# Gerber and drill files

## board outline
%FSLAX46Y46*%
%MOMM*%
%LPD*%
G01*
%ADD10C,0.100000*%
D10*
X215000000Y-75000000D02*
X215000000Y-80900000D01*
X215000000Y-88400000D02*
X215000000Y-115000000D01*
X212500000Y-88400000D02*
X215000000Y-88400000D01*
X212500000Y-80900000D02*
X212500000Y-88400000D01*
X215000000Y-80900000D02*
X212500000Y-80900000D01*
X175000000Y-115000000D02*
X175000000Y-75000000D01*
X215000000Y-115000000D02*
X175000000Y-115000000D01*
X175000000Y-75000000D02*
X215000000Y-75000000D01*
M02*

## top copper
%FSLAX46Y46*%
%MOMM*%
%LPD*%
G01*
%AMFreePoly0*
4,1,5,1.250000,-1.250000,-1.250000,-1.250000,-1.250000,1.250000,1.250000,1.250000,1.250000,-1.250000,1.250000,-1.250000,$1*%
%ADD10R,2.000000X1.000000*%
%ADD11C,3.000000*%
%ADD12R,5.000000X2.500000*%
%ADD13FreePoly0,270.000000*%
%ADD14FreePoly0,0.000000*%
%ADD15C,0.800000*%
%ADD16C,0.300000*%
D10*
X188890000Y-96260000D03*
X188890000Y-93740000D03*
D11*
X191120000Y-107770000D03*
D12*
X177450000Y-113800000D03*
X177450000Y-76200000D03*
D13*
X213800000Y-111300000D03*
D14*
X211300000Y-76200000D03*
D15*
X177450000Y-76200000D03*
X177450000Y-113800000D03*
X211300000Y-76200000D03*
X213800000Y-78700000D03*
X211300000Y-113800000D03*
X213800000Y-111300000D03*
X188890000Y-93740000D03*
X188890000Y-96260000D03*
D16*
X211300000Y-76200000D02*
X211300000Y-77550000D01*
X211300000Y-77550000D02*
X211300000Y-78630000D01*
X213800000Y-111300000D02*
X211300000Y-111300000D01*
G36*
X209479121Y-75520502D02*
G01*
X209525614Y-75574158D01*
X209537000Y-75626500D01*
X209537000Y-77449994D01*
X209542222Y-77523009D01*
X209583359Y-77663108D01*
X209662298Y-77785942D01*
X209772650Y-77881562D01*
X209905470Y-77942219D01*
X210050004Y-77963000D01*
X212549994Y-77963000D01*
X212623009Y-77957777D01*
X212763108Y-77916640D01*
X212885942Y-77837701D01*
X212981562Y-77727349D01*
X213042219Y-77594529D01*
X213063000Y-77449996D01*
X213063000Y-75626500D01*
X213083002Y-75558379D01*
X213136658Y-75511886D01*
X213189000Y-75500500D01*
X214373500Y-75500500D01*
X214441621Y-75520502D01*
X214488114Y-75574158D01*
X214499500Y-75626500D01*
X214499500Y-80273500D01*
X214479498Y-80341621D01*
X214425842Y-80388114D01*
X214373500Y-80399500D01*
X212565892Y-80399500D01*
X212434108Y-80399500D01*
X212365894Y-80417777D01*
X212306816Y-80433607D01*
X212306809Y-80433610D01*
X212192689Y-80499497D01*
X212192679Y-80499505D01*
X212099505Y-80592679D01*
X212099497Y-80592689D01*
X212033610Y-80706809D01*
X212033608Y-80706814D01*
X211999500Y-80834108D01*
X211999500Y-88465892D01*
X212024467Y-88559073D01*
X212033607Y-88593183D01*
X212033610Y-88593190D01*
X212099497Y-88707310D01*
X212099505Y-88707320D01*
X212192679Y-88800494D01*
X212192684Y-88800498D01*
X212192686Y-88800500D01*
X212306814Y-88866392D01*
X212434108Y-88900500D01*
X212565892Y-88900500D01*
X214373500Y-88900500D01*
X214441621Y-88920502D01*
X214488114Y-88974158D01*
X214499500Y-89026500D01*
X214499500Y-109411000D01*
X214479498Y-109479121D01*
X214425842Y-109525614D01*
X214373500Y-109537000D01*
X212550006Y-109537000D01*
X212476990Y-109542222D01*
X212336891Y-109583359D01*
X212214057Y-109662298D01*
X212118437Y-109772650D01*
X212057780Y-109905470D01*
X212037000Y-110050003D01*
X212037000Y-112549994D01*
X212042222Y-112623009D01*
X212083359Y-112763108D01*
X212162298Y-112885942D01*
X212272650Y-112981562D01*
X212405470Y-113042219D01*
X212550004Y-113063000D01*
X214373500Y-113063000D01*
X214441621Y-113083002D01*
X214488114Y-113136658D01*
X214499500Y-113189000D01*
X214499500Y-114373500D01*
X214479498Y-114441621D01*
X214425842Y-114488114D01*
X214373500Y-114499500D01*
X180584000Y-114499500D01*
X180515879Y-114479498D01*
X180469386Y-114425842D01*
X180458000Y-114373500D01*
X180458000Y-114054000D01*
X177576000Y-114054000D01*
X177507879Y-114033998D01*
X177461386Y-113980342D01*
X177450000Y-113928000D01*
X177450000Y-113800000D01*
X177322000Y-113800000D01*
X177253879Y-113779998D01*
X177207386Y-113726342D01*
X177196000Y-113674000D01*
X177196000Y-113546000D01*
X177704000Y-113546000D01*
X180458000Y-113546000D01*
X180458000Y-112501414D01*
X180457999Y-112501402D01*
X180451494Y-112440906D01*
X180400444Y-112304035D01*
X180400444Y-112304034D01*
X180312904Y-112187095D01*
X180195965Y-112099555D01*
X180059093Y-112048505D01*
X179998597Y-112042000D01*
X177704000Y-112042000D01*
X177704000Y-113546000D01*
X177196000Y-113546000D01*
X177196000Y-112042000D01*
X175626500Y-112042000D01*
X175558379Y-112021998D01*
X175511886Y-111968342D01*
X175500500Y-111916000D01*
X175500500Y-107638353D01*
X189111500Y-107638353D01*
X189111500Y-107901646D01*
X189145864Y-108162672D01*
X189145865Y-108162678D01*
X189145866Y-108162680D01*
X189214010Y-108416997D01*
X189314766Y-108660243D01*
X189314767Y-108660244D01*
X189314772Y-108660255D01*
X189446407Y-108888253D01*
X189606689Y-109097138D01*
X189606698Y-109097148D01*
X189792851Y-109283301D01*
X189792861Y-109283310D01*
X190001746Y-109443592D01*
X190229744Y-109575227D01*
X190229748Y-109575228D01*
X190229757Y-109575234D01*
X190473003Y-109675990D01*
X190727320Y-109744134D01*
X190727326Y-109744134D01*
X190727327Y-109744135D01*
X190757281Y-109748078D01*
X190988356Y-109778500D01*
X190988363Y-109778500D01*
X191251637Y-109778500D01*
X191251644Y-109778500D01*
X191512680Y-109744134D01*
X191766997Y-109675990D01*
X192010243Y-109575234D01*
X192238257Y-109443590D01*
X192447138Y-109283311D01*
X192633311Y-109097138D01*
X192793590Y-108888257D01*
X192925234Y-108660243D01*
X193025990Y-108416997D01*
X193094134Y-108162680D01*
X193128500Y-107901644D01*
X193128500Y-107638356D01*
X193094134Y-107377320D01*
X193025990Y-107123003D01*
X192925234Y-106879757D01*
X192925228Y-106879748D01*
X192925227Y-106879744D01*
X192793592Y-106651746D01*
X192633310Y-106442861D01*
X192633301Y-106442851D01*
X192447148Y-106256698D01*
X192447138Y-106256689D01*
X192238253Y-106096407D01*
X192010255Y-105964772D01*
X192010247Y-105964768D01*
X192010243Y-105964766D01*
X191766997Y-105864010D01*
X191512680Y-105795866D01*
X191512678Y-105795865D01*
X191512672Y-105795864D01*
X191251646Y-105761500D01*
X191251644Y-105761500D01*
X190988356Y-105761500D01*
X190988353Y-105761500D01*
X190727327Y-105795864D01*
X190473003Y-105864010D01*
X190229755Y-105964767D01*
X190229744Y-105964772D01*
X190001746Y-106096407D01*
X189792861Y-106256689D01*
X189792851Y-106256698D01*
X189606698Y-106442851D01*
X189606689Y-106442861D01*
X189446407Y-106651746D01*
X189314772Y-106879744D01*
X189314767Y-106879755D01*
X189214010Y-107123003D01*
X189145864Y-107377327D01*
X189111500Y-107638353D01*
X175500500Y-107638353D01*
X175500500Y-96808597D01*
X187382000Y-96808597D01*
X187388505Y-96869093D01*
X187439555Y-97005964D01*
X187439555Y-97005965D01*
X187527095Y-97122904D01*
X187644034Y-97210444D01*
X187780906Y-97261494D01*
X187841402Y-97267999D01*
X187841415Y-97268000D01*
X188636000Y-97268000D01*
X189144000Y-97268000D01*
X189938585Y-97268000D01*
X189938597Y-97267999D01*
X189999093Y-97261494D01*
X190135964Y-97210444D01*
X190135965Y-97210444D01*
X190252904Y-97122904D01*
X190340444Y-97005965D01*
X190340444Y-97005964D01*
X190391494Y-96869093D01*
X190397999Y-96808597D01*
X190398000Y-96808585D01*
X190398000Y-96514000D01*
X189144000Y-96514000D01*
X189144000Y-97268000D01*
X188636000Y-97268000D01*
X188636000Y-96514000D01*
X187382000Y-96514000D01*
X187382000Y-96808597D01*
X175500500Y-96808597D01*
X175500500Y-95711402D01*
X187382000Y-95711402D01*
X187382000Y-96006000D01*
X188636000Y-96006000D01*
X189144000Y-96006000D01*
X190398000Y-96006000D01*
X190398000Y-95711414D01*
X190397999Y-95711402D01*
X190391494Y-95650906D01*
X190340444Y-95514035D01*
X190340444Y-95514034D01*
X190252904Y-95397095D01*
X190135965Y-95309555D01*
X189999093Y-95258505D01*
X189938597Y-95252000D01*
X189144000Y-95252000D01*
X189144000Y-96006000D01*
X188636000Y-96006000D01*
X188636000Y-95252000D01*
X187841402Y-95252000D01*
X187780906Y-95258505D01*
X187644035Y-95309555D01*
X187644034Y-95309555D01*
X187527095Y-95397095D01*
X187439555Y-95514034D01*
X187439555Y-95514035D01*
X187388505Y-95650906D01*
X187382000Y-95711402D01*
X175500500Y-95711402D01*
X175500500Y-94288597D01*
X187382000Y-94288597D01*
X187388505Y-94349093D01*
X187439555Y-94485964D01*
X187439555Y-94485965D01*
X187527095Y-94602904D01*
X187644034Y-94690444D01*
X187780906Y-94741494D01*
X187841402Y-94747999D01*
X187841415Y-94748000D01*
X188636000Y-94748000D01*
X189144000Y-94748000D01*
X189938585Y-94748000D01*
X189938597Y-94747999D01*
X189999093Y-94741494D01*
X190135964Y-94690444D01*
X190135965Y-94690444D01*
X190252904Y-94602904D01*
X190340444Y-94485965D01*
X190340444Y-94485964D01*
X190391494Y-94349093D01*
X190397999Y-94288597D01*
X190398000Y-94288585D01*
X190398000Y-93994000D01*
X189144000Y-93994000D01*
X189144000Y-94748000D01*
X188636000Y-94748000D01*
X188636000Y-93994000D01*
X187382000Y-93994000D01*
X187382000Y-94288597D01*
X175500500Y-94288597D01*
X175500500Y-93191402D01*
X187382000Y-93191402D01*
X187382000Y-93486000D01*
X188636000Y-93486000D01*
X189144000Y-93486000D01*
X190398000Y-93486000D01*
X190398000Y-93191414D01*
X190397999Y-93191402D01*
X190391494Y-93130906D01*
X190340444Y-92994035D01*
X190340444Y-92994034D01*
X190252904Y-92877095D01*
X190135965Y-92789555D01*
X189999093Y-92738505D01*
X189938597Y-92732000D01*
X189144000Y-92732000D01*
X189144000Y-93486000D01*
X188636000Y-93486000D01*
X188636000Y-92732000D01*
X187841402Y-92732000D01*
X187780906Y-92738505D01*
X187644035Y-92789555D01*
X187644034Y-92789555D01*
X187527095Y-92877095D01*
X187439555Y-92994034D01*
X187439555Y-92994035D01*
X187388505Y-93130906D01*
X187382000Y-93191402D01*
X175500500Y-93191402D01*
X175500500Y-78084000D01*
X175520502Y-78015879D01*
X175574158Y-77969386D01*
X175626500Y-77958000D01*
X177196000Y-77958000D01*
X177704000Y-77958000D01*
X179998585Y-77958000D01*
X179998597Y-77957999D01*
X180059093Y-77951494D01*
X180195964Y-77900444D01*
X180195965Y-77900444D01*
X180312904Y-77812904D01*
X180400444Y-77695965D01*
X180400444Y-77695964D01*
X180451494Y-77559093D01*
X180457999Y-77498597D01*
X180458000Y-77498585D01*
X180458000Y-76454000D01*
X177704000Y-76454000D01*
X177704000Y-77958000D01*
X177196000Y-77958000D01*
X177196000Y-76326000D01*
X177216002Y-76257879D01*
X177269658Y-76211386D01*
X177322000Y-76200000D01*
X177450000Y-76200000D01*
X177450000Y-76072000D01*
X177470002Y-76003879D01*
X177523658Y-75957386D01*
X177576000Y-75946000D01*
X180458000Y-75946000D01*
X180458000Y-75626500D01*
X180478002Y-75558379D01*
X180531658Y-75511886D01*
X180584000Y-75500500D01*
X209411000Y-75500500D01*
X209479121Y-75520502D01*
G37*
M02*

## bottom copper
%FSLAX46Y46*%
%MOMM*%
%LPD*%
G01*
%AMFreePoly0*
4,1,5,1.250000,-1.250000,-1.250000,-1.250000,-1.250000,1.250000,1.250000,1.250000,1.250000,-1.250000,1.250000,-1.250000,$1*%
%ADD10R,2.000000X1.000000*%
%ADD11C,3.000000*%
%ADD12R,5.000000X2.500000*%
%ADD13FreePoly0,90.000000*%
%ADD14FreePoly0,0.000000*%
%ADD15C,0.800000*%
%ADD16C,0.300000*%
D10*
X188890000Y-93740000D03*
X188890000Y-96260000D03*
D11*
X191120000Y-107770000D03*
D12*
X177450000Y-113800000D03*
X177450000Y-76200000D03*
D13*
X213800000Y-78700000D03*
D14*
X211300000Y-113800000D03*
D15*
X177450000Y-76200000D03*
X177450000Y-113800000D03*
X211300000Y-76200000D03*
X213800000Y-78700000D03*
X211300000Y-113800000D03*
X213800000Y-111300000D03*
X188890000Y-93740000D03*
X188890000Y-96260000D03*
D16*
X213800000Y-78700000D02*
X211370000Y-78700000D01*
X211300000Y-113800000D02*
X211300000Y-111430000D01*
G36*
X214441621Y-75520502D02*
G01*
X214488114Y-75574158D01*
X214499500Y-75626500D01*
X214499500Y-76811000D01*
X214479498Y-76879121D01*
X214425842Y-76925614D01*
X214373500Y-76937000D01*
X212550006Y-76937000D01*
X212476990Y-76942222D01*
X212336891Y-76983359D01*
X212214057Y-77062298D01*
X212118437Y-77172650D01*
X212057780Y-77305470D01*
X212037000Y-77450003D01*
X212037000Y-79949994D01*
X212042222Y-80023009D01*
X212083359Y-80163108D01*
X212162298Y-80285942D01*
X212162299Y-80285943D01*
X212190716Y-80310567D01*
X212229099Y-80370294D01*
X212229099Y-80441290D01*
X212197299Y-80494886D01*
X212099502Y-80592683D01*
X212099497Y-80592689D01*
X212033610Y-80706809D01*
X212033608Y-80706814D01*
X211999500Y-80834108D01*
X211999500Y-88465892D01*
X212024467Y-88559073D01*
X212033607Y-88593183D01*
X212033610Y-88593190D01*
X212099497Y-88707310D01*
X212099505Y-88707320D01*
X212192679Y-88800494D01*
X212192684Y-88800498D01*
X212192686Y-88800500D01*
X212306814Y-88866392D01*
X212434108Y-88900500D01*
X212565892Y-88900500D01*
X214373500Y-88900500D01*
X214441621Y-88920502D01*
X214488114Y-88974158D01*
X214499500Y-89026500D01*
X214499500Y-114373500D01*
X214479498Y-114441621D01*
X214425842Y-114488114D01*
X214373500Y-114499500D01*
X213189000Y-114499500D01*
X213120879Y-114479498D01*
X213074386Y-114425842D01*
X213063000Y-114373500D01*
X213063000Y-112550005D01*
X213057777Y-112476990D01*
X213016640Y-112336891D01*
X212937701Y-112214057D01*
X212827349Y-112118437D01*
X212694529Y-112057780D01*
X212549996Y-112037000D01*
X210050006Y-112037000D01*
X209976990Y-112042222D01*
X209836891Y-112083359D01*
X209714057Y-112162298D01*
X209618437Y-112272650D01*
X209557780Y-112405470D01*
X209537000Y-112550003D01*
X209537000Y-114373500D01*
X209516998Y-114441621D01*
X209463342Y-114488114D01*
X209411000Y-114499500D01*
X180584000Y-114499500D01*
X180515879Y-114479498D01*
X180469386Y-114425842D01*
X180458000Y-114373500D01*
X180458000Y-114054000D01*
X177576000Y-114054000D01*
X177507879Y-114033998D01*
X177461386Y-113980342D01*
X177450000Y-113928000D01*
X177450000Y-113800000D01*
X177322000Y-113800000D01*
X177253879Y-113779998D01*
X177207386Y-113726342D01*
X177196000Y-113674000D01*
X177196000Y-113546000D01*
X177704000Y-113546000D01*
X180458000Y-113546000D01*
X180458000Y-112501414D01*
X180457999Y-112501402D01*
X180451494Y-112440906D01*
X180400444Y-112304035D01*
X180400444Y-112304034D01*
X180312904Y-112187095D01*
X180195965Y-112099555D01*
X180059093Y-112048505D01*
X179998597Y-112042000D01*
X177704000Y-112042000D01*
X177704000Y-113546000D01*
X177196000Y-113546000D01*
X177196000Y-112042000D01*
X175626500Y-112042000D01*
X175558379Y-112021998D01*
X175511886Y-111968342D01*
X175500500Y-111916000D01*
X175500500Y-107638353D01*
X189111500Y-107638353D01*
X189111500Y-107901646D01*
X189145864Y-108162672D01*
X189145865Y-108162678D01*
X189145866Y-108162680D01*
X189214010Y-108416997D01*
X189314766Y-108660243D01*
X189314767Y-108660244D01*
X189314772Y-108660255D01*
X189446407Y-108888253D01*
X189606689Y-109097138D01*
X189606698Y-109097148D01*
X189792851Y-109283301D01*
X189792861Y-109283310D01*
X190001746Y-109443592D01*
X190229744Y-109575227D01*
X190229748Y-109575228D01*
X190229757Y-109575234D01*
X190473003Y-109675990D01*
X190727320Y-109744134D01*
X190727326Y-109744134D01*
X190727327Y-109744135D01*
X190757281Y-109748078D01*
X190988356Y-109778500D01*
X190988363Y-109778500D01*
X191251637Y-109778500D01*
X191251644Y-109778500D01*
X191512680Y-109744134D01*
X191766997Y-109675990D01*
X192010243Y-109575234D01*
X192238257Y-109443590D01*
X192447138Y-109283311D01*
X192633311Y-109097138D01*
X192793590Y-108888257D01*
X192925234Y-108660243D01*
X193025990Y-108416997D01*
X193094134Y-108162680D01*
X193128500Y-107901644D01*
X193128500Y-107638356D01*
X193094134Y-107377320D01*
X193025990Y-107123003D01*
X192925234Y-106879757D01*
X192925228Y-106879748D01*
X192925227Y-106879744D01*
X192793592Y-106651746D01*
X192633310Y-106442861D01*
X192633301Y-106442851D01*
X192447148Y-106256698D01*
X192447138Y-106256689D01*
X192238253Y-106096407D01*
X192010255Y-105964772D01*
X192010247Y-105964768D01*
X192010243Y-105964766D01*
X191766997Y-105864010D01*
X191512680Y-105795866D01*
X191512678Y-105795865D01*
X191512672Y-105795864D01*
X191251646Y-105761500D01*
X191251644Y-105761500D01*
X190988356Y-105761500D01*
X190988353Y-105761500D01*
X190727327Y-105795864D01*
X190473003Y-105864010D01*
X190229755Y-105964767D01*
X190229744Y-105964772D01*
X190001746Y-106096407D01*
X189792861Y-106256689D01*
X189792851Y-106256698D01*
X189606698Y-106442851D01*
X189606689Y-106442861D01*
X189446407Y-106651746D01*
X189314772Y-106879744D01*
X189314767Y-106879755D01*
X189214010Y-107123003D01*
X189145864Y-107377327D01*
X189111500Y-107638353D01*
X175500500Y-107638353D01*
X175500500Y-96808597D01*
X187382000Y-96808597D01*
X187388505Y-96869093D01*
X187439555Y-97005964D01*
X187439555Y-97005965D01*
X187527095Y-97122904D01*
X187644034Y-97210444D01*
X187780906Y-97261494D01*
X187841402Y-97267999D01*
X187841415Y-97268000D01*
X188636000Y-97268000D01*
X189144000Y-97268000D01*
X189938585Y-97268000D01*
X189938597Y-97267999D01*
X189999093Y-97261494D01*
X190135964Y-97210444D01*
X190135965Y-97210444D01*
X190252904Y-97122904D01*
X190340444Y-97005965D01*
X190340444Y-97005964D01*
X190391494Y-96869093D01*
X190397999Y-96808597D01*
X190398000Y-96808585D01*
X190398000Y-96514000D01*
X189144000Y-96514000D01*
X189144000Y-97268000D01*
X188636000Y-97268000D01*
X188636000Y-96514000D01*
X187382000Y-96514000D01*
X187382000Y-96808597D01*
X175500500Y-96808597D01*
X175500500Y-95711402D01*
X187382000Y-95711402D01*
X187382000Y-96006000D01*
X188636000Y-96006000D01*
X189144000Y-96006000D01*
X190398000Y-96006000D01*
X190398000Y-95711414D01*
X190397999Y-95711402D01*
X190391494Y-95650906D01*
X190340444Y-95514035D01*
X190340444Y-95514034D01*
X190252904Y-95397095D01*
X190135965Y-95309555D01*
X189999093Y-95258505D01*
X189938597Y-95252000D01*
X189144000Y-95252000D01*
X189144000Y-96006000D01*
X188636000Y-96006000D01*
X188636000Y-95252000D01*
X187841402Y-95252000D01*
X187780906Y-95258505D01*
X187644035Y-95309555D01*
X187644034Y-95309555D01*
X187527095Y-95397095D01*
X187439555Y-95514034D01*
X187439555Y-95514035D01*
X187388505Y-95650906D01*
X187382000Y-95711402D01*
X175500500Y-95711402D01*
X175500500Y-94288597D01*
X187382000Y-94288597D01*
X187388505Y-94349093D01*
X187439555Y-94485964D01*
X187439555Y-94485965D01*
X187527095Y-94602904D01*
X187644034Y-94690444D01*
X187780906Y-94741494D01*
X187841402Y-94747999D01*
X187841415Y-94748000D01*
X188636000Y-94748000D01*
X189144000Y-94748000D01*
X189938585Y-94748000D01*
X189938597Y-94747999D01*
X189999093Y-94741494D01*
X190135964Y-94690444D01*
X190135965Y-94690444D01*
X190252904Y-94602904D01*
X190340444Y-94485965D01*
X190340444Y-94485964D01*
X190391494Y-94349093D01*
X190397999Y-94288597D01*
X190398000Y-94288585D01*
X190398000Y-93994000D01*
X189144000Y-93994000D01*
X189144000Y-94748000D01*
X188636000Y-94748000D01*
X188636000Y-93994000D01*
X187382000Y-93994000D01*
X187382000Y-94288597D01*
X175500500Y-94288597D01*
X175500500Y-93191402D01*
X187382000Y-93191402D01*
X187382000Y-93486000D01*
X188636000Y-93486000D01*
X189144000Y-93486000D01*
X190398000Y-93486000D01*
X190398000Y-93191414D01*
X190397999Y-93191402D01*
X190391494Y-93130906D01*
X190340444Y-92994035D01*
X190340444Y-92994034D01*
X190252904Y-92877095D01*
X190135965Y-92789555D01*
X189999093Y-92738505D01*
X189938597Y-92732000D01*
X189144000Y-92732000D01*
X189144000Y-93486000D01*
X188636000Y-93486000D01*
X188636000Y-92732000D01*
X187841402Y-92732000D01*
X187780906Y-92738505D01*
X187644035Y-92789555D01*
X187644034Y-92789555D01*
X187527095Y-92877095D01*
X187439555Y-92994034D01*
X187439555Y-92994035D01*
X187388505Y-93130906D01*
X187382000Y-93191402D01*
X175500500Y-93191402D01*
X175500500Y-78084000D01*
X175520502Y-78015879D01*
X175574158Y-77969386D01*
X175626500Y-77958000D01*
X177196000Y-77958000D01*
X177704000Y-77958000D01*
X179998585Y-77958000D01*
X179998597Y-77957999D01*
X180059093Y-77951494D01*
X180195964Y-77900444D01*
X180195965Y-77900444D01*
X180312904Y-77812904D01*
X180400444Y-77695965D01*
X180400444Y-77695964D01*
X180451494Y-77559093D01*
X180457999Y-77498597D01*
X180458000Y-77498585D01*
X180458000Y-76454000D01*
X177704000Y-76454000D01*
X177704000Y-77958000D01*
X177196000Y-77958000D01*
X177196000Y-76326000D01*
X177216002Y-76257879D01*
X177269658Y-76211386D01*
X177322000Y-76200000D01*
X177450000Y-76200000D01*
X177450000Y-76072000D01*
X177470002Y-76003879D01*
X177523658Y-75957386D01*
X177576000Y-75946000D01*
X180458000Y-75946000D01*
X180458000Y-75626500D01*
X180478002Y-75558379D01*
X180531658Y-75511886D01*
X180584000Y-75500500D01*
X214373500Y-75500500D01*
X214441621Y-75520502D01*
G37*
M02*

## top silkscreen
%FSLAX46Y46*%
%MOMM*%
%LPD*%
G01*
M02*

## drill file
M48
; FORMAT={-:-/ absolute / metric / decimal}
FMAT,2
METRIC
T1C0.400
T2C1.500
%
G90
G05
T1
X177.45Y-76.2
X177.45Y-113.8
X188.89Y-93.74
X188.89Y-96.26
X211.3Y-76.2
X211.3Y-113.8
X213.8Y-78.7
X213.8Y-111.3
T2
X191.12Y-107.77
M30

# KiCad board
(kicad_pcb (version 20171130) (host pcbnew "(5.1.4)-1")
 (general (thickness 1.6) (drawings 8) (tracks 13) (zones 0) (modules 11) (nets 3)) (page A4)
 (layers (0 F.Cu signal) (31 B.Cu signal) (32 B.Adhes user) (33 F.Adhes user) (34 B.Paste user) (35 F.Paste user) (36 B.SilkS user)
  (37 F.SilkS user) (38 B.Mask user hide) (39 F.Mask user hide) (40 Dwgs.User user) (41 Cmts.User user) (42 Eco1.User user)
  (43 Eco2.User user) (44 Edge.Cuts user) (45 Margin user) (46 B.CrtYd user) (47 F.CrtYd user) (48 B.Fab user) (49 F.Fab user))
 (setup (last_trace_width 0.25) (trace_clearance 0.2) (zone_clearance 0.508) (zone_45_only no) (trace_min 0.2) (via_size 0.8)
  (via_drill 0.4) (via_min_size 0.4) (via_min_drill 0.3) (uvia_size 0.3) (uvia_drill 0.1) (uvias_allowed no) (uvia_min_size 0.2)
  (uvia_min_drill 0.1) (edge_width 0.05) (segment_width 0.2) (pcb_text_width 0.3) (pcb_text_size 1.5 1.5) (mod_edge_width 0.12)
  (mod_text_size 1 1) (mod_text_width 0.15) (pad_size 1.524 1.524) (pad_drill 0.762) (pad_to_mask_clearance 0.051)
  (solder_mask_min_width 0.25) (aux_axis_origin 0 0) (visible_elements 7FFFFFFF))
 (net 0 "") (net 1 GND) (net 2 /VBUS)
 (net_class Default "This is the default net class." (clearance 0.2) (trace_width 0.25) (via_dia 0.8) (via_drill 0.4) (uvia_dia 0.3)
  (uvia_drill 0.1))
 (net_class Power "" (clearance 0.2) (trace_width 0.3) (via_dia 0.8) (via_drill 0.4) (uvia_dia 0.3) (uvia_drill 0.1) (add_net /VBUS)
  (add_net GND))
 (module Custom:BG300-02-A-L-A (layer B.Cu) (at 190.39 95 90)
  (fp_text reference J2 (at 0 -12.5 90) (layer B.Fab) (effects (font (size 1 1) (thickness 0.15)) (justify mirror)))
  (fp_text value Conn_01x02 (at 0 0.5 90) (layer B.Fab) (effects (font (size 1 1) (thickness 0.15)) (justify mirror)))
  (pad 2 smd rect (at 1.26 -1.5 90) (size 1 2) (layers B.Cu B.Paste B.Mask) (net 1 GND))
  (pad 1 smd rect (at -1.26 -1.5 90) (size 1 2) (layers B.Cu B.Paste B.Mask) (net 1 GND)))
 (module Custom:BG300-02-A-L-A (layer F.Cu) (at 190.39 95 270)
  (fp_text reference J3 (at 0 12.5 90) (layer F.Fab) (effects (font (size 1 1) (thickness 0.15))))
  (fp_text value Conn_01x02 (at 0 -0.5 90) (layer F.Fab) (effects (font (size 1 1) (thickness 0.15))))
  (pad 2 smd rect (at 1.26 1.5 270) (size 1 2) (layers F.Cu F.Paste F.Mask) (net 1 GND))
  (pad 1 smd rect (at -1.26 1.5 270) (size 1 2) (layers F.Cu F.Paste F.Mask) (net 1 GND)))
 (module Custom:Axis (layer F.Cu) (at 191.12 107.77)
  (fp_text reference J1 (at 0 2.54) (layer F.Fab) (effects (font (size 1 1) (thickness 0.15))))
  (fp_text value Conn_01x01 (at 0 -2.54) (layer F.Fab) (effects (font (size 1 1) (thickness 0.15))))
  (pad 1 thru_hole circle (at 0 0) (size 3 3) (drill 1.5) (layers *.Cu *.Mask) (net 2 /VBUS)))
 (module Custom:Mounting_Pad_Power (layer B.Cu) (at 177.45 113.8 90)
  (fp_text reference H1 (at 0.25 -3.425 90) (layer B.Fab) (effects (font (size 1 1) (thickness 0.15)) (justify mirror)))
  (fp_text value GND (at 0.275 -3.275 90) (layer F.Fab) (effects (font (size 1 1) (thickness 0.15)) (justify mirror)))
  (pad 1 smd rect (at 0 0 90) (size 2.5 5) (layers B.Cu B.Paste B.Mask) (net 1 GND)))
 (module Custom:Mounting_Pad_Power (layer F.Cu) (at 177.45 113.8 90)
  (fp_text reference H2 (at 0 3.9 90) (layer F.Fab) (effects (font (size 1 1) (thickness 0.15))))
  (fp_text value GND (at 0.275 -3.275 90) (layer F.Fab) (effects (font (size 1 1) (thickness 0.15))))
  (pad 1 smd rect (at 0 0 90) (size 2.5 5) (layers F.Cu F.Paste F.Mask) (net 1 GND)))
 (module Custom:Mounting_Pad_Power (layer F.Cu) (at 177.45 76.2 270)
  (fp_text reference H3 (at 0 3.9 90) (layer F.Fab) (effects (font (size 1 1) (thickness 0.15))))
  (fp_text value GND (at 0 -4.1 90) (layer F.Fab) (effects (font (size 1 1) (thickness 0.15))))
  (pad 1 smd rect (at 0 0 270) (size 2.5 5) (layers F.Cu F.Paste F.Mask) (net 1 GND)))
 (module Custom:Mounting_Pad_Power (layer B.Cu) (at 177.45 76.2 90)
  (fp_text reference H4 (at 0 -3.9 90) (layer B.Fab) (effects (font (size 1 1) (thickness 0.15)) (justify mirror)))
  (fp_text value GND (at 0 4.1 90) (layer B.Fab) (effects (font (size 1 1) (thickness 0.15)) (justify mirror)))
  (pad 1 smd rect (at 0 0 90) (size 2.5 5) (layers B.Cu B.Paste B.Mask) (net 1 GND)))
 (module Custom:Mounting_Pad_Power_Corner (layer F.Cu) (at 213.8 111.3 270)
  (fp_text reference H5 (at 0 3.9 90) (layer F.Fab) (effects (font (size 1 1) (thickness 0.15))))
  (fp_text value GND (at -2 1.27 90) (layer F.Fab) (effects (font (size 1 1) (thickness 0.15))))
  (pad 1 smd custom (at 0 0 270) (size 2.5 2.5) (layers F.Cu F.Paste F.Mask) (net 1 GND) (zone_connect 0)
   (options (clearance outline) (anchor rect)) (primitives)))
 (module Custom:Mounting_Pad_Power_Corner (layer B.Cu) (at 213.8 78.7 90)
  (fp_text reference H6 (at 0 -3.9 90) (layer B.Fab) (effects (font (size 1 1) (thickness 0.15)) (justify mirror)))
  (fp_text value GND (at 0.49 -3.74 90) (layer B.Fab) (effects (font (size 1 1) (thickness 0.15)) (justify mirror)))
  (pad 1 smd custom (at 0 0 90) (size 2.5 2.5) (layers B.Cu B.Paste B.Mask) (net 1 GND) (zone_connect 0)
   (options (clearance outline) (anchor rect)) (primitives)))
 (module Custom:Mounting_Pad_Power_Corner (layer F.Cu) (at 211.3 76.2)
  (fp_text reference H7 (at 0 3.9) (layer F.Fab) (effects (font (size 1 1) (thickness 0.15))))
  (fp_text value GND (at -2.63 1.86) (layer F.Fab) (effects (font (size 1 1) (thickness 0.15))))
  (pad 1 smd custom (at 0 0) (size 2.5 2.5) (layers F.Cu F.Paste F.Mask) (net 1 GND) (zone_connect 0)
   (options (clearance outline) (anchor rect)) (primitives)))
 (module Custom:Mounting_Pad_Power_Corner (layer B.Cu) (at 211.3 113.8)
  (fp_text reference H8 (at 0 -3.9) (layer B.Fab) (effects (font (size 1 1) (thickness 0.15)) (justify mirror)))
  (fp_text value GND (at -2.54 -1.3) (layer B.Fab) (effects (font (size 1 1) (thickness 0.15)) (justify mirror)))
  (pad 1 smd custom (at 0 0) (size 2.5 2.5) (layers B.Cu B.Paste B.Mask) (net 1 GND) (zone_connect 0)
   (options (clearance outline) (anchor rect)) (primitives)))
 (gr_line (start 215 75) (end 215 80.9) (layer Edge.Cuts) (width 0.1))
 (gr_line (start 215 88.4) (end 215 115) (layer Edge.Cuts) (width 0.1))
 (gr_line (start 212.5 88.4) (end 215 88.4) (layer Edge.Cuts) (width 0.1))
 (gr_line (start 212.5 80.9) (end 212.5 88.4) (layer Edge.Cuts) (width 0.1))
 (gr_line (start 215 80.9) (end 212.5 80.9) (layer Edge.Cuts) (width 0.1))
 (gr_line (start 175 115) (end 175 75) (layer Edge.Cuts) (width 0.1))
 (gr_line (start 215 115) (end 175 115) (layer Edge.Cuts) (width 0.1))
 (gr_line (start 175 75) (end 215 75) (layer Edge.Cuts) (width 0.1))
 (via (at 177.45 76.2) (size 0.8) (drill 0.4) (layers F.Cu B.Cu) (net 1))
 (via (at 177.45 113.8) (size 0.8) (drill 0.4) (layers F.Cu B.Cu) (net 1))
 (via (at 211.3 76.2) (size 0.8) (drill 0.4) (layers F.Cu B.Cu) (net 1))
 (via (at 213.8 78.7) (size 0.8) (drill 0.4) (layers F.Cu B.Cu) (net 1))
 (segment (start 213.8 78.7) (end 211.37 78.7) (width 0.3) (layer B.Cu) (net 1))
 (segment (start 211.3 76.2) (end 211.3 77.55) (width 0.3) (layer F.Cu) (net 1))
 (segment (start 211.3 77.55) (end 211.3 78.63) (width 0.3) (layer F.Cu) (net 1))
 (via (at 211.3 113.8) (size 0.8) (drill 0.4) (layers F.Cu B.Cu) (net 1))
 (segment (start 211.3 113.8) (end 211.3 111.43) (width 0.3) (layer B.Cu) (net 1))
 (via (at 213.8 111.3) (size 0.8) (drill 0.4) (layers F.Cu B.Cu) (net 1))
 (segment (start 213.8 111.3) (end 211.3 111.3) (width 0.3) (layer F.Cu) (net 1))
 (via (at 188.89 93.74) (size 0.8) (drill 0.4) (layers F.Cu B.Cu) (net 1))
 (via (at 188.89 96.26) (size 0.8) (drill 0.4) (layers F.Cu B.Cu) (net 1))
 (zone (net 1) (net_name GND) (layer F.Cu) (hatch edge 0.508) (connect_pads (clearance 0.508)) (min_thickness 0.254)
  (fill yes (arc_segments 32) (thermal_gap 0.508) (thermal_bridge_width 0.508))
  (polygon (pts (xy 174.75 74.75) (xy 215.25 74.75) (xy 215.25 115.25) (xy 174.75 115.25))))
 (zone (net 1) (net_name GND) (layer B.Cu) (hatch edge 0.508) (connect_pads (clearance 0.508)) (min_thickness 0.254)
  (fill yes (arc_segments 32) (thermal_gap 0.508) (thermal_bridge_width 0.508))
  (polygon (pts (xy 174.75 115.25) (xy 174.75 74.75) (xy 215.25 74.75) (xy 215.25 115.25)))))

